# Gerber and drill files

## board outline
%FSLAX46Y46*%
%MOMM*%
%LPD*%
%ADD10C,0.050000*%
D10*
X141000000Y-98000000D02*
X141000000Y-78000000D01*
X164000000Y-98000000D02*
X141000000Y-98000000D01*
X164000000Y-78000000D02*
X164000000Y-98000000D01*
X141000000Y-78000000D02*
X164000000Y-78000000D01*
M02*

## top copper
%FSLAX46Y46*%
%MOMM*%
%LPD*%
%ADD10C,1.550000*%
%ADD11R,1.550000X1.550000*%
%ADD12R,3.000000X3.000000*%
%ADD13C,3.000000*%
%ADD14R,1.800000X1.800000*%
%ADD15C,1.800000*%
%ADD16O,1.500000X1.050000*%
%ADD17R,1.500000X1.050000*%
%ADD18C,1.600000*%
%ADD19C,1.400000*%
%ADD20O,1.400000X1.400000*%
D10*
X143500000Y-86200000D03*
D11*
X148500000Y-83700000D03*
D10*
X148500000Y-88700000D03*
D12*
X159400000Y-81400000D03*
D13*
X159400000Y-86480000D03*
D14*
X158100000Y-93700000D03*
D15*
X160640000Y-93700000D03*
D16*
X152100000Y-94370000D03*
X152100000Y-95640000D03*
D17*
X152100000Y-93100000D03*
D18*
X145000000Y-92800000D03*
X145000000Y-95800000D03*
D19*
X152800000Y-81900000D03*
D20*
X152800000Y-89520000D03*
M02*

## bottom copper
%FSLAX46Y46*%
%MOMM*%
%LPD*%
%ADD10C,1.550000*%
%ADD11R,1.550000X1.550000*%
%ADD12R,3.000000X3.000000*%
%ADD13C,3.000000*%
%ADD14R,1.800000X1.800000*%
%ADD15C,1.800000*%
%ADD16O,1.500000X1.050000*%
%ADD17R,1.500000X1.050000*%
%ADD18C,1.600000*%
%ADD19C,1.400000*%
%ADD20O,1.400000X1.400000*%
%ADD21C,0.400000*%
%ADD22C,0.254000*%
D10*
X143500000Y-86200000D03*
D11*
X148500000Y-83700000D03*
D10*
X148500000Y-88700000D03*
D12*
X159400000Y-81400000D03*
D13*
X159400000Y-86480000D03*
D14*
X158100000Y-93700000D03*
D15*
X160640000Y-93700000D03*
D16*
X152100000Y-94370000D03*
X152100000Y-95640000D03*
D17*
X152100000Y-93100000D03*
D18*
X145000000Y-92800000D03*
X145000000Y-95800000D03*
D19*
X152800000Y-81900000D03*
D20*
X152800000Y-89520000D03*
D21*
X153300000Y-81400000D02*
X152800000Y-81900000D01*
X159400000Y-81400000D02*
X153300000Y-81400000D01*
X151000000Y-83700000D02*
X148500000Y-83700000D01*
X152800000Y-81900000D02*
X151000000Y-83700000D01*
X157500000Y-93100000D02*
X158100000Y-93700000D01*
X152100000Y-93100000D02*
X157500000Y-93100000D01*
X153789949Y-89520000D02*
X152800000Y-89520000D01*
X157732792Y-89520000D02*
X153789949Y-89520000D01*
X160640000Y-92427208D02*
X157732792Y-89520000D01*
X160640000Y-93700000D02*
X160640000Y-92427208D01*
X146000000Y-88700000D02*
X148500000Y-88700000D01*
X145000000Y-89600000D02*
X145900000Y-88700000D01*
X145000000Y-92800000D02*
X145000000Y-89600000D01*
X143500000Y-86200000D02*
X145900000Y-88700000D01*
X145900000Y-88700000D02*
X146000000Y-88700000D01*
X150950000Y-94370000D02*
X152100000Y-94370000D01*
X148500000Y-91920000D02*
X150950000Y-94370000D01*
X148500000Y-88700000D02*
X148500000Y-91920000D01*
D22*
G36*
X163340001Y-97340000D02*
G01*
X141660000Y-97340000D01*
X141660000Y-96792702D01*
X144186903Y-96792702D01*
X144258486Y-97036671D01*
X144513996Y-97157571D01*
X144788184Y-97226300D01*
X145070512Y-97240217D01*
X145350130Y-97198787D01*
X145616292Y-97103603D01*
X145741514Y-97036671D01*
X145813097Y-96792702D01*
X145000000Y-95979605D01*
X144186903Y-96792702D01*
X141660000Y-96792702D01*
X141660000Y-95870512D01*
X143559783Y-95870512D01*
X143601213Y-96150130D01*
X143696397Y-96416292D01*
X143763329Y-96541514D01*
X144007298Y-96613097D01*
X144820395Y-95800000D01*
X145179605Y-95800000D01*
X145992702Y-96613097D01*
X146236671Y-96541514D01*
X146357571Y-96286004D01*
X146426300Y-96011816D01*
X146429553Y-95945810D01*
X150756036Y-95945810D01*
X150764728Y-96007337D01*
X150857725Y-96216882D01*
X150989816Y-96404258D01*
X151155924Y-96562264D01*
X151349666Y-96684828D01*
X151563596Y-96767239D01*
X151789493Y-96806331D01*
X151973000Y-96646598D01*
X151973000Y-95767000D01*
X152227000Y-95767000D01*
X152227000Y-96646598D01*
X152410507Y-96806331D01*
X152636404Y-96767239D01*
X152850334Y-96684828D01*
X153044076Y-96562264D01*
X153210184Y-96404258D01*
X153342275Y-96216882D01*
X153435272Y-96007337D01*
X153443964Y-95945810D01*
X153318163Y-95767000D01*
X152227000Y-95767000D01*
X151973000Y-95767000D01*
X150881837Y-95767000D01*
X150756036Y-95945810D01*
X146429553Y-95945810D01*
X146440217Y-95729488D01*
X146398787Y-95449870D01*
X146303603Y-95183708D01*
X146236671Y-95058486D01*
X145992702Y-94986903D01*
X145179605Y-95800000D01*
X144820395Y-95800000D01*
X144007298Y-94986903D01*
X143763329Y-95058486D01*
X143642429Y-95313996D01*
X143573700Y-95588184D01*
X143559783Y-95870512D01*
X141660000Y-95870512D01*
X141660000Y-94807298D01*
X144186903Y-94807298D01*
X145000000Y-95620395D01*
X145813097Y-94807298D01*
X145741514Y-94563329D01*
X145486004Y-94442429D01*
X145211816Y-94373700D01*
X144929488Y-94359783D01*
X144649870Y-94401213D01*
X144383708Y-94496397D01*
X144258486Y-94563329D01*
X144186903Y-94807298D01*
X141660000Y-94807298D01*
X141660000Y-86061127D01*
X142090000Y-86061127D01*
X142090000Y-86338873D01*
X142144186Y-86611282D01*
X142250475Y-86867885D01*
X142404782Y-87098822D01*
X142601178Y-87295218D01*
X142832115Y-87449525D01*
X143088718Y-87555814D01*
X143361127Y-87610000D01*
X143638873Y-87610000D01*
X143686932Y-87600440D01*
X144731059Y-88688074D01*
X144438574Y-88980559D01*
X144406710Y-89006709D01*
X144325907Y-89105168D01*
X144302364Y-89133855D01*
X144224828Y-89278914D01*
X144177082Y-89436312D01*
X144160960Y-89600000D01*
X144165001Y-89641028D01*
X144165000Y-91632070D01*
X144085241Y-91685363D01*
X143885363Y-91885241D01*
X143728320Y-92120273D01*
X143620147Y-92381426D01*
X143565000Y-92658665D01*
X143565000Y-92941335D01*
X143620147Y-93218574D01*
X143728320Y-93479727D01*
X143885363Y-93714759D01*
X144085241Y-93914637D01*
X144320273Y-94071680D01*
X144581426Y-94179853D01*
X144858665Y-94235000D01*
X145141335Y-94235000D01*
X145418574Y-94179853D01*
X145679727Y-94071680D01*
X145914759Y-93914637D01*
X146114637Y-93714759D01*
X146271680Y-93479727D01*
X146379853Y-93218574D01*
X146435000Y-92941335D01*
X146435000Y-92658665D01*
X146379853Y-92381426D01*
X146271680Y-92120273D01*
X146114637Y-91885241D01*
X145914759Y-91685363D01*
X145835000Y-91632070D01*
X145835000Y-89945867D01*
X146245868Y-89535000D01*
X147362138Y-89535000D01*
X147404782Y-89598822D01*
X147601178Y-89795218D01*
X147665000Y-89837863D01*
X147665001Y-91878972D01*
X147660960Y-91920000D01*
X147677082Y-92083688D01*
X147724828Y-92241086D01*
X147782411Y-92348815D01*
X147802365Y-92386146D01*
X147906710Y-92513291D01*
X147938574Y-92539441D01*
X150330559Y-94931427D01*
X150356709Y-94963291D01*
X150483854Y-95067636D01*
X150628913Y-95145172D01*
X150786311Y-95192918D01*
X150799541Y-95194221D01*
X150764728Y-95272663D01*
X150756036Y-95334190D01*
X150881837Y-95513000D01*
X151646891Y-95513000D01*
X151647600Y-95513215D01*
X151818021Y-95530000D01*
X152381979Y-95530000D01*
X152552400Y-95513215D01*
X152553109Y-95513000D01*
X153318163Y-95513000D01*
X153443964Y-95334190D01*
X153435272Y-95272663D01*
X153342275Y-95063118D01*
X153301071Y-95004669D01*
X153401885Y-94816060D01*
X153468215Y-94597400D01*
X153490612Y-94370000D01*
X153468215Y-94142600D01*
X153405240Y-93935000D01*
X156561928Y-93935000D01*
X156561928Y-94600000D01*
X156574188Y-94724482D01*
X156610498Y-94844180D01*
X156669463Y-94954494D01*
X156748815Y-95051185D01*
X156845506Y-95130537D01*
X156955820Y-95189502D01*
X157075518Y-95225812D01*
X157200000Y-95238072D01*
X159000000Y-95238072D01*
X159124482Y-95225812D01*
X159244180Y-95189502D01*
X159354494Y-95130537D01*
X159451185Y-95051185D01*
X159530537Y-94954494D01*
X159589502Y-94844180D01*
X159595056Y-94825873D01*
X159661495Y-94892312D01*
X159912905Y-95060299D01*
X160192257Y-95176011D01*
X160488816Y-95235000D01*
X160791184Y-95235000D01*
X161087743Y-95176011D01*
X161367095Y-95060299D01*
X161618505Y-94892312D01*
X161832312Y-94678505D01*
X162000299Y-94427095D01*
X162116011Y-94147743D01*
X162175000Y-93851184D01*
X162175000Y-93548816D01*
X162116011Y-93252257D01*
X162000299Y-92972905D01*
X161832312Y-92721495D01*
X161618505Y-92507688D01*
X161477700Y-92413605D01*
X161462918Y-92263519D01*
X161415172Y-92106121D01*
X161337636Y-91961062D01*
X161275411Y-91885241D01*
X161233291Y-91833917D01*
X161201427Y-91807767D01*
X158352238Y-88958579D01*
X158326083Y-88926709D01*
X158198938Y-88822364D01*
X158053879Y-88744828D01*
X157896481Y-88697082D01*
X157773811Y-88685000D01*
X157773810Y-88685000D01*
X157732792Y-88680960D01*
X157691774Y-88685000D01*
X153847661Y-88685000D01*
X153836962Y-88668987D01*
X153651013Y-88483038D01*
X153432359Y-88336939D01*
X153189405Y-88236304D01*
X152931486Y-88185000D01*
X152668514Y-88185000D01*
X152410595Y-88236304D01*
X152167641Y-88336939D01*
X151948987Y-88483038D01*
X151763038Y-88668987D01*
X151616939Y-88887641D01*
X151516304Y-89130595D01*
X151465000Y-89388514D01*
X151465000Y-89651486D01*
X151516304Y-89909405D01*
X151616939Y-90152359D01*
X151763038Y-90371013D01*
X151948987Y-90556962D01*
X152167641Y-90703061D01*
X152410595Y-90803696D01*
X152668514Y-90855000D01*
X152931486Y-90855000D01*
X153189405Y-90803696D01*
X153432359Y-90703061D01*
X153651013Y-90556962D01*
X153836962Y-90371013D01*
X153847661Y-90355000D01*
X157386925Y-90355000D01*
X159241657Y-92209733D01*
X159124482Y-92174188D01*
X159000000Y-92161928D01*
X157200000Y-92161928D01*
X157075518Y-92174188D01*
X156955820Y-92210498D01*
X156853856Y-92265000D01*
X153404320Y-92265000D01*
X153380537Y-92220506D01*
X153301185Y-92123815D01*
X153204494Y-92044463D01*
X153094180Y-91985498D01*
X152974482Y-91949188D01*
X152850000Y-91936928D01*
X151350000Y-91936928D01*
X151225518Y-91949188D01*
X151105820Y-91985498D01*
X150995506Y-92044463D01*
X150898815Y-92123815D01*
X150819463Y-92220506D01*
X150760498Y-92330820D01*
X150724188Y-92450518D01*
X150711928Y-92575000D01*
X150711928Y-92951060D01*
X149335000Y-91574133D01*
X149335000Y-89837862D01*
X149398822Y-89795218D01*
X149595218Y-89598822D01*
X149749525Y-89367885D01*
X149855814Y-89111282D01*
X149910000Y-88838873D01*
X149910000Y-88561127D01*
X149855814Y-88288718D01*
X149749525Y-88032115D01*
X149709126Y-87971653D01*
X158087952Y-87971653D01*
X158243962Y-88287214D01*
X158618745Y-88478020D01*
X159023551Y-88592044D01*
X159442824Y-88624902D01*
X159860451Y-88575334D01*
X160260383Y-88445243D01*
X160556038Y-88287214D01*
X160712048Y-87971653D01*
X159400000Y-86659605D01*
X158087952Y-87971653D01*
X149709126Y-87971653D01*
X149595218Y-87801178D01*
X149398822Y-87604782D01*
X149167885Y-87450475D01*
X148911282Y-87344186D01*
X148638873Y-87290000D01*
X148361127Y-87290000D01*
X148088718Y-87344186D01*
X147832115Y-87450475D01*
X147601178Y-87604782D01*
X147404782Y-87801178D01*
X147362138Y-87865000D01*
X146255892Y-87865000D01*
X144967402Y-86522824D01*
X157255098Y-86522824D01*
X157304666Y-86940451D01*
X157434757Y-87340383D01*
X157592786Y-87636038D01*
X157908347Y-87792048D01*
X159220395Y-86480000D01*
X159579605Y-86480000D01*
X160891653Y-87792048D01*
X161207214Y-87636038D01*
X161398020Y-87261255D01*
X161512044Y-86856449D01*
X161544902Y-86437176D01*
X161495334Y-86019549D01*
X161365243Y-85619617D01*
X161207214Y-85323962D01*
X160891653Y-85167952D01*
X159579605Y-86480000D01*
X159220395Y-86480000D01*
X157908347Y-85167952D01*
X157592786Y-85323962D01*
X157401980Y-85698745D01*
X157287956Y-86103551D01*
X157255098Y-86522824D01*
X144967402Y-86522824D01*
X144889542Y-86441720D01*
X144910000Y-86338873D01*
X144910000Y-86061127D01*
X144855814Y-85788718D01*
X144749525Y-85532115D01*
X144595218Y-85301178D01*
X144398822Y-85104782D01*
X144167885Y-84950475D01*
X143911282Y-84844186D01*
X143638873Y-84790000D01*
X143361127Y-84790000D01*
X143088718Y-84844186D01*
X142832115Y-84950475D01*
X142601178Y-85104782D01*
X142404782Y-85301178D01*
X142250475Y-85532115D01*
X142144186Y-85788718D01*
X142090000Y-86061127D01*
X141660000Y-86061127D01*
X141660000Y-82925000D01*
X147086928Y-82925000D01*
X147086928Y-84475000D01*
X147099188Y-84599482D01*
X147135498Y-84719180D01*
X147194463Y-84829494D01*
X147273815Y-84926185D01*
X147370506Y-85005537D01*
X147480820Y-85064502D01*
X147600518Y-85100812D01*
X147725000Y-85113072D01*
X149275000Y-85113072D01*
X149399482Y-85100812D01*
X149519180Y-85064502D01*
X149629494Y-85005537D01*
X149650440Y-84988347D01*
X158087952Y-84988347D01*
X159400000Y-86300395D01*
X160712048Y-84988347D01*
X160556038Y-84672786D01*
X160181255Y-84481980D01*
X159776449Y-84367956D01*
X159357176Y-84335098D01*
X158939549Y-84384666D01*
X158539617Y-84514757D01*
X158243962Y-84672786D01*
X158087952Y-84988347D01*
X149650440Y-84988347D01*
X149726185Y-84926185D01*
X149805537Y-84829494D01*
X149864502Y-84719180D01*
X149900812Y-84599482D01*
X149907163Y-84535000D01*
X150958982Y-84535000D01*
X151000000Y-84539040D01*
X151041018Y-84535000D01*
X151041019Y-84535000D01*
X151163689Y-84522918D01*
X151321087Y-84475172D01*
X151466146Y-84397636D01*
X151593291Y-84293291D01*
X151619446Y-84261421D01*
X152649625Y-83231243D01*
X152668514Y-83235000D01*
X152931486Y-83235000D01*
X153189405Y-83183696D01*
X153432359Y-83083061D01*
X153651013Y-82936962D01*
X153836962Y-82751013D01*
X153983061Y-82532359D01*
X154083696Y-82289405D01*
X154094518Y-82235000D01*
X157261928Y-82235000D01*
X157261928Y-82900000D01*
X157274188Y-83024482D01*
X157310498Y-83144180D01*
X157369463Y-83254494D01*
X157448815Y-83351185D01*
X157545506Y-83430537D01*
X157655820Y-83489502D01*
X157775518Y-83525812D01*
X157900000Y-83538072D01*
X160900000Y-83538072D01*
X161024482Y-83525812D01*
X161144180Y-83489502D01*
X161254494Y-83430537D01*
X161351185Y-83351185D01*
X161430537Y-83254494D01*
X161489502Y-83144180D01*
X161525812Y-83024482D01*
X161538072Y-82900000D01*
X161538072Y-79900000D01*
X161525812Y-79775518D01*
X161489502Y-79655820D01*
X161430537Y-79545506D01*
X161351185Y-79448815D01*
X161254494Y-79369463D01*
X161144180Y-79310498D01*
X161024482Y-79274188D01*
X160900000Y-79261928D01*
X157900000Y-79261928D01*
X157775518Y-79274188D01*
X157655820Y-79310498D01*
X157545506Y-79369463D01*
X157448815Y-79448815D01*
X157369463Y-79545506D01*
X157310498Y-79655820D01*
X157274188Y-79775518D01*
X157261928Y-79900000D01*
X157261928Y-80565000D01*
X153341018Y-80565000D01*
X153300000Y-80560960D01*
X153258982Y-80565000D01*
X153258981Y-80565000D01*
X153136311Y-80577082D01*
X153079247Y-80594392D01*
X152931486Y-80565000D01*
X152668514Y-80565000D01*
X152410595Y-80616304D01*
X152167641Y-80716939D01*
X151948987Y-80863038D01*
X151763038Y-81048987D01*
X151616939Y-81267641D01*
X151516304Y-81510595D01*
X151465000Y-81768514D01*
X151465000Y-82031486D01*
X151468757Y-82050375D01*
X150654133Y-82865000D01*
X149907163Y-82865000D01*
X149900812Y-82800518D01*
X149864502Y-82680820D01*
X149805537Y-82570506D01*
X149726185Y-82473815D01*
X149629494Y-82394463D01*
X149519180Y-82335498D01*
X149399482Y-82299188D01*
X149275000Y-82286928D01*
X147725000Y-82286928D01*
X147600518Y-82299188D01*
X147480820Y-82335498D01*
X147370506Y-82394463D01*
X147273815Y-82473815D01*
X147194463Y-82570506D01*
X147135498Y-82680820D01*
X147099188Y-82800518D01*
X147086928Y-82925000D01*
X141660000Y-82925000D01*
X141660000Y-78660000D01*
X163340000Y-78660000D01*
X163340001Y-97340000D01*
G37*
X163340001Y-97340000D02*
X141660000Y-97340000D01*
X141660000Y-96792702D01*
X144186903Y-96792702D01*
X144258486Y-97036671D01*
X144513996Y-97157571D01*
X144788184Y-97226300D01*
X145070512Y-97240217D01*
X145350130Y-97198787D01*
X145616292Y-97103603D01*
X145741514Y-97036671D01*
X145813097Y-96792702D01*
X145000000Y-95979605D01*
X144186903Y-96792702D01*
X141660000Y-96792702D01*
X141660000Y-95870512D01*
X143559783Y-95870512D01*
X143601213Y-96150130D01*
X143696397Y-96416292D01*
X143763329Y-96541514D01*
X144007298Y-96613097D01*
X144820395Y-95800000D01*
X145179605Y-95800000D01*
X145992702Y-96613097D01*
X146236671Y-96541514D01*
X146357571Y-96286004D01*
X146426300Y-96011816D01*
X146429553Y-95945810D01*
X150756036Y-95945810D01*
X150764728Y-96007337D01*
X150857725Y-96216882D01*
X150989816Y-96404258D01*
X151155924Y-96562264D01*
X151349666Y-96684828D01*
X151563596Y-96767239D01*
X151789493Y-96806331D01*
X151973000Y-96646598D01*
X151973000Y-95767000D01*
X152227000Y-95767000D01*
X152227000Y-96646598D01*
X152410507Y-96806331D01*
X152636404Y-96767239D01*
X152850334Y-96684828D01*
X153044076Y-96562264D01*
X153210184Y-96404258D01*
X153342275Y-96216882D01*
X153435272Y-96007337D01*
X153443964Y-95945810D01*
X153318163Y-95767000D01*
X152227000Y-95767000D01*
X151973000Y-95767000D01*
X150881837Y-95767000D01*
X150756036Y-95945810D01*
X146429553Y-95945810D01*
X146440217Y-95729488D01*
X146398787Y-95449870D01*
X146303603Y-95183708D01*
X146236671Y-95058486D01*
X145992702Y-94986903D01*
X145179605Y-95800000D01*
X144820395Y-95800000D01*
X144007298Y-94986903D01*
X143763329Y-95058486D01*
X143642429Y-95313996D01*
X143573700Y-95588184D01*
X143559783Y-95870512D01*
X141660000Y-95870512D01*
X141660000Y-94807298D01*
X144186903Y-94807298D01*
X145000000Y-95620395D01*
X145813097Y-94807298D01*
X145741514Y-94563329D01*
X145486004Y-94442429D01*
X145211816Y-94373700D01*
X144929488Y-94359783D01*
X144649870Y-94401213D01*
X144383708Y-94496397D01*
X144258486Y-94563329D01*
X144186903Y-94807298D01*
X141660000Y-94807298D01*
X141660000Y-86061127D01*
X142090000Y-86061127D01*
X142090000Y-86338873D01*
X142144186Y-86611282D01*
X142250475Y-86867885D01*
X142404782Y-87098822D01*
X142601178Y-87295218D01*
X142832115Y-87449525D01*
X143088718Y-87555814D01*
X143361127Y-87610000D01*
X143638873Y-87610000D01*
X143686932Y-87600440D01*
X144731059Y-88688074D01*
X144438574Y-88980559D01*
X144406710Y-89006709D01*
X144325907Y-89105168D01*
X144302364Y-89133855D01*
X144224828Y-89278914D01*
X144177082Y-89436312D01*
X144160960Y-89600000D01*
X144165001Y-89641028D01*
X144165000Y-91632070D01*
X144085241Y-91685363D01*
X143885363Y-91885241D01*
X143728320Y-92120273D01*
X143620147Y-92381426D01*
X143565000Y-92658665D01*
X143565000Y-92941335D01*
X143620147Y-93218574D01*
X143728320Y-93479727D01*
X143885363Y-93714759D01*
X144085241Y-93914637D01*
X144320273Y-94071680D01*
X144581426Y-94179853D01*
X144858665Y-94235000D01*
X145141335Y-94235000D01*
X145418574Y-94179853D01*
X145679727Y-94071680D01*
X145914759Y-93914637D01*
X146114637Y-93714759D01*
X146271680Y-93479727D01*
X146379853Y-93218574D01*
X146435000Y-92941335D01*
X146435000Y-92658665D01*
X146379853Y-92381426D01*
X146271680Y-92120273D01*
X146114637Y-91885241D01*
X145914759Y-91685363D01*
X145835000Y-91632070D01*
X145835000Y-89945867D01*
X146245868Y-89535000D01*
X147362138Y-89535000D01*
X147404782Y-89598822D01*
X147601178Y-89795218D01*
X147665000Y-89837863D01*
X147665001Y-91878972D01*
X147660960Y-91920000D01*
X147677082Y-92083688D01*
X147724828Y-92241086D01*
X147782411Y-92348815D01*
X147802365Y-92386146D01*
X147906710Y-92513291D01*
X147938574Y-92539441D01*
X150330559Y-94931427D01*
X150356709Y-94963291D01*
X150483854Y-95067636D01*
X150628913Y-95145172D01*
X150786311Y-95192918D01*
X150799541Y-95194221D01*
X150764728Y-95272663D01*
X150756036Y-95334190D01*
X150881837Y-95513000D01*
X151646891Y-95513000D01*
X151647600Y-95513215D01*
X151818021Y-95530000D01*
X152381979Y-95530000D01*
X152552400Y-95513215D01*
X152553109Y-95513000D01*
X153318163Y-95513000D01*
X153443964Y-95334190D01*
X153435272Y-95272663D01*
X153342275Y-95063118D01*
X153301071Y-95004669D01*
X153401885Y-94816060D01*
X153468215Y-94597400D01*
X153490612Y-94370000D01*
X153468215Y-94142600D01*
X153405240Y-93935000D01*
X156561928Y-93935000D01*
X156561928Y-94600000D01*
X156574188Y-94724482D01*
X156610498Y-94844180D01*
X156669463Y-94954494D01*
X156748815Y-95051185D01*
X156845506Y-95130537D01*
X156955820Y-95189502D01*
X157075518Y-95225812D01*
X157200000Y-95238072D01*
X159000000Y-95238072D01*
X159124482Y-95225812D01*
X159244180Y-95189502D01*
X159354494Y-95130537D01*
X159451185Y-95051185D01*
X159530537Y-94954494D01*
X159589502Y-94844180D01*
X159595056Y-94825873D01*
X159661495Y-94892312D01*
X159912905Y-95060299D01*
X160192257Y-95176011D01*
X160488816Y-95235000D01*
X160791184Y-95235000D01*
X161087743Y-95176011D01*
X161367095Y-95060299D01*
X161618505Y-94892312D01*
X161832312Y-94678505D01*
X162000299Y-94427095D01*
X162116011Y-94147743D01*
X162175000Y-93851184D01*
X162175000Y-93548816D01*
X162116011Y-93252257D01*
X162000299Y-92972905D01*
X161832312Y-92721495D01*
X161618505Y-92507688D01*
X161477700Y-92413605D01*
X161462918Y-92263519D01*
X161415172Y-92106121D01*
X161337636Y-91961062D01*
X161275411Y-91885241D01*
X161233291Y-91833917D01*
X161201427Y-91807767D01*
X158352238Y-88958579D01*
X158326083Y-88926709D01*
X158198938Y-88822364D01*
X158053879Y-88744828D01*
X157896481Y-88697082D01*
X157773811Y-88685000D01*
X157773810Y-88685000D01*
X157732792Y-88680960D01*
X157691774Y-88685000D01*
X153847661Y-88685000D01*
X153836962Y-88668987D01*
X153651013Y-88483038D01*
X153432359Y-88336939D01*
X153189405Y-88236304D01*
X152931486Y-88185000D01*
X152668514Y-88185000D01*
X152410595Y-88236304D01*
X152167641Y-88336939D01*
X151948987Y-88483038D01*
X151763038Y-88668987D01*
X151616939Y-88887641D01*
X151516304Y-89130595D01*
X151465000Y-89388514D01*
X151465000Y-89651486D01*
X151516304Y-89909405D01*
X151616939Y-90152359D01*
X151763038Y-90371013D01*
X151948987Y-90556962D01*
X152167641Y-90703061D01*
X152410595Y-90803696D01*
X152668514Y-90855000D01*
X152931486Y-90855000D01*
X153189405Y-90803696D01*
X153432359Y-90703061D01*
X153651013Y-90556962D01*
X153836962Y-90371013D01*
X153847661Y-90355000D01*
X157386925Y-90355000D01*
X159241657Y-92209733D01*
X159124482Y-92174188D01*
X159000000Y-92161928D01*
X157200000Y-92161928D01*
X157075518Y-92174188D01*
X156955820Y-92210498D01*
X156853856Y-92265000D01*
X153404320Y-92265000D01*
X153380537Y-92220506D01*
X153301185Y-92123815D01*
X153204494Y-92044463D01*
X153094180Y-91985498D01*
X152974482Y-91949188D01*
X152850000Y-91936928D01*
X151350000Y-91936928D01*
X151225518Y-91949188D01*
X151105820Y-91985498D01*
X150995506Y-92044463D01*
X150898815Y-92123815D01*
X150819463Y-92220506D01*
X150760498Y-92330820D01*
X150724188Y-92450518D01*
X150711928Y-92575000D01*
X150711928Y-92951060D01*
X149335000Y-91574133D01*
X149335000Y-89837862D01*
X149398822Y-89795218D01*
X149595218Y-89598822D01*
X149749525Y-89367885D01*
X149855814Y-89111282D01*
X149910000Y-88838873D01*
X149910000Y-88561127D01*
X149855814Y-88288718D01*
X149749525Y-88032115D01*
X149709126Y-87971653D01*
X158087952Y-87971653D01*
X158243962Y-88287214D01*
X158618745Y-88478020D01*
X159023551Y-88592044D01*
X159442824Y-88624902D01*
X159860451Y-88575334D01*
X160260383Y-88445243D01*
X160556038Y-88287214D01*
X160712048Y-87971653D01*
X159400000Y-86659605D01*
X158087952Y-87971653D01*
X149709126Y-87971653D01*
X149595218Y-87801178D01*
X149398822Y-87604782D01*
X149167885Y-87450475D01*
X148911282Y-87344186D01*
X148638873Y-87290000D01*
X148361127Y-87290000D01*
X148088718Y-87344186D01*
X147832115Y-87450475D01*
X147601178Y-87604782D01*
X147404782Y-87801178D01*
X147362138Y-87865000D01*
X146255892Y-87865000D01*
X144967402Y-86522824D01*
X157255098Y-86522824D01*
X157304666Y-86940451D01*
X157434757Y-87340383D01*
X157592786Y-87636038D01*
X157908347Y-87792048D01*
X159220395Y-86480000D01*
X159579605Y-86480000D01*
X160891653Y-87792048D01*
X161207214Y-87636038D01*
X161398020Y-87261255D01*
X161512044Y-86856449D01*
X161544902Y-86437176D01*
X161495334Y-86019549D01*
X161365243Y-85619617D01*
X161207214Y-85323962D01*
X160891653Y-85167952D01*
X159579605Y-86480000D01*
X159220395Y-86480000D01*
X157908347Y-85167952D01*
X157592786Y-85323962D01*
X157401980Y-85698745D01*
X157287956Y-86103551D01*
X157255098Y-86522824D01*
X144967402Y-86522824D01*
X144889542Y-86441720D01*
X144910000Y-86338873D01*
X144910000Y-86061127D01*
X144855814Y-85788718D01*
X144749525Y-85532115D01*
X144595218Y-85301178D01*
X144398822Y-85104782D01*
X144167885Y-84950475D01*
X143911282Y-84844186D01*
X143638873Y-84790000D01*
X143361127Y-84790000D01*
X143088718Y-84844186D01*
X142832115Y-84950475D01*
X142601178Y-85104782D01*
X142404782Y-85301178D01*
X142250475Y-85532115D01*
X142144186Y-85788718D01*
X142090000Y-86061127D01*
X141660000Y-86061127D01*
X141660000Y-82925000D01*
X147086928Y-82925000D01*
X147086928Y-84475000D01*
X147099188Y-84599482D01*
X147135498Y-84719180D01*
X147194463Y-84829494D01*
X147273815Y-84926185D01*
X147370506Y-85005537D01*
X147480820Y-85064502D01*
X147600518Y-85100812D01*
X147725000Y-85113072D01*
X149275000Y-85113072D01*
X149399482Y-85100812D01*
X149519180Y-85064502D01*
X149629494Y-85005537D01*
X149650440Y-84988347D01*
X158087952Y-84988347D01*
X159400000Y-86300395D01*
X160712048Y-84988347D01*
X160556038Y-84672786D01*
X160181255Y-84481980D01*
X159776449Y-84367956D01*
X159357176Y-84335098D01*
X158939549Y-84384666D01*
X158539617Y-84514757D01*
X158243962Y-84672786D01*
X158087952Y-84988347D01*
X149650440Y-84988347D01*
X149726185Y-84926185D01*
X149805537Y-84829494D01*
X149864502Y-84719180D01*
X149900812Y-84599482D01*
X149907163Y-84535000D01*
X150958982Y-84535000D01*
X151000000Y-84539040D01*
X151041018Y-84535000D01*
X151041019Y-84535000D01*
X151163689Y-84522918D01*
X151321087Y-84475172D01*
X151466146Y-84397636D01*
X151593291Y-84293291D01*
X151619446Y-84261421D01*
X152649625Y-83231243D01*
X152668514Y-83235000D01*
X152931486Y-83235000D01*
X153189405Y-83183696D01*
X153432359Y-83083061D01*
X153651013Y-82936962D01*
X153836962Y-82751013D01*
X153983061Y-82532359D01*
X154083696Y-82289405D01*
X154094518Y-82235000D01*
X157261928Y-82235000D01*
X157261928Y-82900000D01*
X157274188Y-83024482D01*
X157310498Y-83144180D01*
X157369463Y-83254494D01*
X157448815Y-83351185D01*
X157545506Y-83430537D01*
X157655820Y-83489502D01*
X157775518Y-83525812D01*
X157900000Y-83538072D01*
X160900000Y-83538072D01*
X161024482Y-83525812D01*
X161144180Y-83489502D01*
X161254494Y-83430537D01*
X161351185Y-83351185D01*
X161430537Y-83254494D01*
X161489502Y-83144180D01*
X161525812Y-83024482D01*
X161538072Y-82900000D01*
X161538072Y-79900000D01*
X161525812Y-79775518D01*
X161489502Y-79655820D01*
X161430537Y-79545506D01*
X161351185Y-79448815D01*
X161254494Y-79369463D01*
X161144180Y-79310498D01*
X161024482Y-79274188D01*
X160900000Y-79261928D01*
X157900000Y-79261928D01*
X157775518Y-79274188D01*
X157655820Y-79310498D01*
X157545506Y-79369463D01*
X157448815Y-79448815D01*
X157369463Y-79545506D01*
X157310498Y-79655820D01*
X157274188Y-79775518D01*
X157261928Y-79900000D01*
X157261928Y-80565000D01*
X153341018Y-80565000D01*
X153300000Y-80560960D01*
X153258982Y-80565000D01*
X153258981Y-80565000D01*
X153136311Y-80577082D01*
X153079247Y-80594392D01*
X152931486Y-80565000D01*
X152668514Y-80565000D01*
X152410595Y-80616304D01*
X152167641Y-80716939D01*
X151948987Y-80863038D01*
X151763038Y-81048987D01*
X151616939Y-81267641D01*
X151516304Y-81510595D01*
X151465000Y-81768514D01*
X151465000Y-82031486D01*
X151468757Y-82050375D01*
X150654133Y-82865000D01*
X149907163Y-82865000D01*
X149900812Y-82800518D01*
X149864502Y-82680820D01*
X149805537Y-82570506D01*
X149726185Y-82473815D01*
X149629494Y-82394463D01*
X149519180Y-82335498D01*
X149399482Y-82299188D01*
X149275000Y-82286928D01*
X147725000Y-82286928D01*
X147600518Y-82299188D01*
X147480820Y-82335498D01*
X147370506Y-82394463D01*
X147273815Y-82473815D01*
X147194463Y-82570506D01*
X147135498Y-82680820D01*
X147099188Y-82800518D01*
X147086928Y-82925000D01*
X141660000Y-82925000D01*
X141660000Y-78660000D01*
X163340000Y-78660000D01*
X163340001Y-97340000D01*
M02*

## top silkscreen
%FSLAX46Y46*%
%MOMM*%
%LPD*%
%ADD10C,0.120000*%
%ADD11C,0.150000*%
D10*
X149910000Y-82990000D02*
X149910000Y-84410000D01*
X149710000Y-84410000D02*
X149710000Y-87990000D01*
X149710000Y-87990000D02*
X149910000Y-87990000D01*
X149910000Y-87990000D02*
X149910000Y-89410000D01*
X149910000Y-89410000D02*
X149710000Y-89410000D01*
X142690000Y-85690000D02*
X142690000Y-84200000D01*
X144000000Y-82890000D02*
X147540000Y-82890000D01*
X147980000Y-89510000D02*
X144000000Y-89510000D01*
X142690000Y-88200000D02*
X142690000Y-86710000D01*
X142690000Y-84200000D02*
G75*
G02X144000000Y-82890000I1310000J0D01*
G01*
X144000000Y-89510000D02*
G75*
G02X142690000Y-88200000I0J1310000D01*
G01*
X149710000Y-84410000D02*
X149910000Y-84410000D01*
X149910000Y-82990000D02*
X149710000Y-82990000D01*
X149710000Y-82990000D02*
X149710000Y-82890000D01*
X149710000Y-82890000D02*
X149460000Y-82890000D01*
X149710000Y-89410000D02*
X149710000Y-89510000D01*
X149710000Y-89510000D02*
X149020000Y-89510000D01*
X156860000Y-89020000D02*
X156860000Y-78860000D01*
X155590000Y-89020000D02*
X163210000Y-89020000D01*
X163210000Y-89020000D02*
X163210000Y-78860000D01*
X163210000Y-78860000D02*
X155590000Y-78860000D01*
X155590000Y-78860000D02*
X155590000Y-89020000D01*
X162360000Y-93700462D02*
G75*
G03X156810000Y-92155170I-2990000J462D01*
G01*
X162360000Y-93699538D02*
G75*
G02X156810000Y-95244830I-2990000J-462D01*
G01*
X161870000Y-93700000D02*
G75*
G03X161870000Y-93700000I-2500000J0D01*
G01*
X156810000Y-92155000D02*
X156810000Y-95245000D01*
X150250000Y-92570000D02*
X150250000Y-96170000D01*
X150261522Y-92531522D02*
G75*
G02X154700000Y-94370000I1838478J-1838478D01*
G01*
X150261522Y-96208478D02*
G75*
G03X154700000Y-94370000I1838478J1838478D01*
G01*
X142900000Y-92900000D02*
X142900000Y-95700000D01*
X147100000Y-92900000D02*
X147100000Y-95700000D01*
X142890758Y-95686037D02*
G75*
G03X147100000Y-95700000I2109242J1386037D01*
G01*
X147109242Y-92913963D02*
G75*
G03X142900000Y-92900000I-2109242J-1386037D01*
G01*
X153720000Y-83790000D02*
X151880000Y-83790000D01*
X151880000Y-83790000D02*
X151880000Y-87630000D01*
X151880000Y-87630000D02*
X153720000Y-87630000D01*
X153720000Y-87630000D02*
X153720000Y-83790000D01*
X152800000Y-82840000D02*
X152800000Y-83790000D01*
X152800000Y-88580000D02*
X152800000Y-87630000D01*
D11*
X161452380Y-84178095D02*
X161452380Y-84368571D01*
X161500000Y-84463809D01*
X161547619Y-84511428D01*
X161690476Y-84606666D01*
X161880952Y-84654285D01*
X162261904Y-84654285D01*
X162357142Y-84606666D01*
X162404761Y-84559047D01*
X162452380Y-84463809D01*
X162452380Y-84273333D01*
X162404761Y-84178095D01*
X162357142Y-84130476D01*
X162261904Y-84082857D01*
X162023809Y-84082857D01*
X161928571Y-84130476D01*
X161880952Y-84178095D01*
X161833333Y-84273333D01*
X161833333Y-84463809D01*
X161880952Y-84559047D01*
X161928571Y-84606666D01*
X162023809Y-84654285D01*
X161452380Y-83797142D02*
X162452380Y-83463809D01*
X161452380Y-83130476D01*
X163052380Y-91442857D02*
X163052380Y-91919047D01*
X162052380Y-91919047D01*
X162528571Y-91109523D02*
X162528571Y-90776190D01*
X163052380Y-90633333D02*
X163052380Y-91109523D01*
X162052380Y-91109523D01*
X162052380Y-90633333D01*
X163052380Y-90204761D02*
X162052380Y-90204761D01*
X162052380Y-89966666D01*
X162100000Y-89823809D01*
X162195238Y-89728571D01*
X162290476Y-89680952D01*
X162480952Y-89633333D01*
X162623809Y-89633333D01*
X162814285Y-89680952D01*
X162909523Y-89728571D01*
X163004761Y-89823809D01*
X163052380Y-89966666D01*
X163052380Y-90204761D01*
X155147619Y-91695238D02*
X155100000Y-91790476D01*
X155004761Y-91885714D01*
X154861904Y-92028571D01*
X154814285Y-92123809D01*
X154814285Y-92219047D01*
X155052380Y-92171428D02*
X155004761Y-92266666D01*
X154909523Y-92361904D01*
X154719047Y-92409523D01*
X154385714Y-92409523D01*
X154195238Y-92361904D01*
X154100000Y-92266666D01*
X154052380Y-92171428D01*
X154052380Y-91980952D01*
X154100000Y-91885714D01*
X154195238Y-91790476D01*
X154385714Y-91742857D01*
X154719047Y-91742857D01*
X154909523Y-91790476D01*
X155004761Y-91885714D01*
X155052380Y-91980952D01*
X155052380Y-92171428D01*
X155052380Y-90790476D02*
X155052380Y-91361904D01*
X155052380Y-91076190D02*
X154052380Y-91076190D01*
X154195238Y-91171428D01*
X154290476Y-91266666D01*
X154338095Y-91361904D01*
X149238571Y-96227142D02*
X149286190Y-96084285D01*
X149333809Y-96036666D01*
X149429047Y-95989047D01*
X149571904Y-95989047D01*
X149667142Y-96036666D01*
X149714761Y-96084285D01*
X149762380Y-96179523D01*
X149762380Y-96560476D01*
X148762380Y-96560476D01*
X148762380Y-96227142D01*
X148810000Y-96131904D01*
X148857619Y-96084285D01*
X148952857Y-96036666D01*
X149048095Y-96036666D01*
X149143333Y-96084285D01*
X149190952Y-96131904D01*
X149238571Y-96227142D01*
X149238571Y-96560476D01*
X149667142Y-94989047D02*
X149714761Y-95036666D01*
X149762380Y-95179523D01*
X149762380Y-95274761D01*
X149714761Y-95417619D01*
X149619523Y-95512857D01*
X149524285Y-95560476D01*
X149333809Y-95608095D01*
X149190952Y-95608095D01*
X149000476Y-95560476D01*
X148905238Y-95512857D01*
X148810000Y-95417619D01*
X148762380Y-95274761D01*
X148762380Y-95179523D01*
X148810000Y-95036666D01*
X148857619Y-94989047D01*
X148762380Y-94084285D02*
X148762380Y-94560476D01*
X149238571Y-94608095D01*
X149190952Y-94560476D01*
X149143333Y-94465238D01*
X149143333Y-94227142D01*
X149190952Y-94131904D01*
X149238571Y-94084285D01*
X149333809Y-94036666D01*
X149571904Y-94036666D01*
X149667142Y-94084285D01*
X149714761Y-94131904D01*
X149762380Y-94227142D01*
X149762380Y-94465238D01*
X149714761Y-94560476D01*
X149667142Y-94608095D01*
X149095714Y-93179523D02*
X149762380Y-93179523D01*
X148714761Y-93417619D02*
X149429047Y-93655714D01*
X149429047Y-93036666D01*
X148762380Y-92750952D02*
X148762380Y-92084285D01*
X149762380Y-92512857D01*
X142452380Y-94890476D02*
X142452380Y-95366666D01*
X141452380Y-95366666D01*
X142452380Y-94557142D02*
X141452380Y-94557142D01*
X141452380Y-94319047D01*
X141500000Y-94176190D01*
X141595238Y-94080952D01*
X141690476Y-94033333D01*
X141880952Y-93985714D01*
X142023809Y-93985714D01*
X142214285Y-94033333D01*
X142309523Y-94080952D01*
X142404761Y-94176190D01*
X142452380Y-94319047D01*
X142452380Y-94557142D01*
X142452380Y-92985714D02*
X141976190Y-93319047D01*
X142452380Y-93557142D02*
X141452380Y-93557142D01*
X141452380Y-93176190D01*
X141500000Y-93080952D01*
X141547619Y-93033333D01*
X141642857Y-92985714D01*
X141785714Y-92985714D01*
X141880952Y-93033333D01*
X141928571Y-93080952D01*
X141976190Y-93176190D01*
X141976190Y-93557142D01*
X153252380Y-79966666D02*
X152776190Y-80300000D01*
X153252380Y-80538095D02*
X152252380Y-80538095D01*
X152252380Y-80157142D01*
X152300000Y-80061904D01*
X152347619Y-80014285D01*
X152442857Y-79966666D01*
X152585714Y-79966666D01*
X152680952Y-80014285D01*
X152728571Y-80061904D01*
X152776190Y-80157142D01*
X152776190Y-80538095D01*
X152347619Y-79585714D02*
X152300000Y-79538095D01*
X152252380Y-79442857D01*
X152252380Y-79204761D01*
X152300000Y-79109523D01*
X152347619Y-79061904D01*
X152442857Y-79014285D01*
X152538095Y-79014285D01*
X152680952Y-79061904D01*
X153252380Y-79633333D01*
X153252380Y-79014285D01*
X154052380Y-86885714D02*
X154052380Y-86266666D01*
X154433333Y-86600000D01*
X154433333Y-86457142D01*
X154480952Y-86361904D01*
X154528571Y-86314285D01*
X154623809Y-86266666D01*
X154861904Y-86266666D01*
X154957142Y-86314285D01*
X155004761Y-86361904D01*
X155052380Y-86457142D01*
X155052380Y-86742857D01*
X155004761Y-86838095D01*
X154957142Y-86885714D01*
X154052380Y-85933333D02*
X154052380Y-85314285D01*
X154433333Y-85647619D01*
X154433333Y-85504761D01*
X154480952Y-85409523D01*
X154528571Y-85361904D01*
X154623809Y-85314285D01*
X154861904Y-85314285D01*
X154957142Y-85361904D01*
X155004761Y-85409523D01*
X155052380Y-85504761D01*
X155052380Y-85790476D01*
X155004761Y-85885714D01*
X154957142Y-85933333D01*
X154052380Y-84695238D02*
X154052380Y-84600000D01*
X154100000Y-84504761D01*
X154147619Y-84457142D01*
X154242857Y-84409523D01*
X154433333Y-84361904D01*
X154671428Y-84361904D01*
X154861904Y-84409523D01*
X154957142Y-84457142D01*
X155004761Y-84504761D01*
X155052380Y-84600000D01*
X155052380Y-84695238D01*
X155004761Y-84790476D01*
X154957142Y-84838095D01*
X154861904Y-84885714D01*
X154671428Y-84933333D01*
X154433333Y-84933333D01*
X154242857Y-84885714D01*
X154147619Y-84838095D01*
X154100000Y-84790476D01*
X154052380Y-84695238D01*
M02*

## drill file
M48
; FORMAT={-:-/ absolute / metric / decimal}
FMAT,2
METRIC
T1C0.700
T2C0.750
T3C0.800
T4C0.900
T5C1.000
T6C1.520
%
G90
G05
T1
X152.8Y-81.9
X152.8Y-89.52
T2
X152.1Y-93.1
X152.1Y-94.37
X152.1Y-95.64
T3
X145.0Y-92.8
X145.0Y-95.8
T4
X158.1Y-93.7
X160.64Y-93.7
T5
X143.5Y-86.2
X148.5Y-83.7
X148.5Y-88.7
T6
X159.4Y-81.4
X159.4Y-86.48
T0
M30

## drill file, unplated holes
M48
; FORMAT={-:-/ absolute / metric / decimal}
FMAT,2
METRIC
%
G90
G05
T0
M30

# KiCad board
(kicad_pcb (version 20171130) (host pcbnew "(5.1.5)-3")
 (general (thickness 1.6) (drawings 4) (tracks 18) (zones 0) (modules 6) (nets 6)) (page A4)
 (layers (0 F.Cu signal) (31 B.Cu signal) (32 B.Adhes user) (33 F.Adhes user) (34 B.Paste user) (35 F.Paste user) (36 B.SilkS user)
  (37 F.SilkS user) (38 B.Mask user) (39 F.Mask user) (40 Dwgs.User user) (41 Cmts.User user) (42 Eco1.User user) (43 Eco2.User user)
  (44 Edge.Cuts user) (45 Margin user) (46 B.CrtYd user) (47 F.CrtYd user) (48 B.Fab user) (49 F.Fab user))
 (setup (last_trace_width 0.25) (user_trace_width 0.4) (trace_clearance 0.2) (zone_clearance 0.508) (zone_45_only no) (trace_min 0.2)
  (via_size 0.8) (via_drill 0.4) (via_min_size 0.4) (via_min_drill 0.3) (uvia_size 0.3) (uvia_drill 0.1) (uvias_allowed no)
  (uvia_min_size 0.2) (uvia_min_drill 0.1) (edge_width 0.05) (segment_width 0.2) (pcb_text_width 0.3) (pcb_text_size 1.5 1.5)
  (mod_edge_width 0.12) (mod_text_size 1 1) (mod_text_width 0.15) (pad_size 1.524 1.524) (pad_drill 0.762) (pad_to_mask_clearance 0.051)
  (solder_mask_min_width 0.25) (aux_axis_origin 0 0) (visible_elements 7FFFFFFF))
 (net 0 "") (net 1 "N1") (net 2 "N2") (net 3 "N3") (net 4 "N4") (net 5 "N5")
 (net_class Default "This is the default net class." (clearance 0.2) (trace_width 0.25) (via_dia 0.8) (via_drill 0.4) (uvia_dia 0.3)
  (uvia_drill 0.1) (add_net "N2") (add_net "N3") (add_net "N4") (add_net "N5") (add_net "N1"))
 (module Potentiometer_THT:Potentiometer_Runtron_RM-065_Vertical (layer F.Cu) (at 148.5 83.7 270)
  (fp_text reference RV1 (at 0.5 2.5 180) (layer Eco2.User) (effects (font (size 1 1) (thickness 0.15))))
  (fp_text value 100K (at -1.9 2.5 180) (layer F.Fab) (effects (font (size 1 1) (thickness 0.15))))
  (fp_line (start -0.71 -1.41) (end 0.71 -1.41) (layer F.SilkS) (width 0.12))
  (fp_line (start 0.71 -1.21) (end 4.29 -1.21) (layer F.SilkS) (width 0.12))
  (fp_line (start 4.29 -1.21) (end 4.29 -1.41) (layer F.SilkS) (width 0.12))
  (fp_line (start 4.29 -1.41) (end 5.71 -1.41) (layer F.SilkS) (width 0.12))
  (fp_line (start 5.71 -1.41) (end 5.71 -1.21) (layer F.SilkS) (width 0.12))
  (fp_line (start 1.99 5.81) (end 0.5 5.81) (layer F.SilkS) (width 0.12))
  (fp_line (start -0.81 4.5) (end -0.81 0.96) (layer F.SilkS) (width 0.12))
  (fp_line (start 5.81 0.52) (end 5.81 4.5) (layer F.SilkS) (width 0.12))
  (fp_line (start 4.5 5.81) (end 3.01 5.81) (layer F.SilkS) (width 0.12))
  (fp_arc (start 0.5 4.5) (end -0.81 4.5) (angle -90) (layer F.SilkS) (width 0.12))
  (fp_arc (start 4.5 4.5) (end 4.5 5.81) (angle -90) (layer F.SilkS) (width 0.12))
  (fp_line (start 0.71 -1.21) (end 0.71 -1.41) (layer F.SilkS) (width 0.12))
  (fp_line (start -0.71 -1.41) (end -0.71 -1.21) (layer F.SilkS) (width 0.12))
  (fp_line (start -0.71 -1.21) (end -0.81 -1.21) (layer F.SilkS) (width 0.12))
  (fp_line (start -0.81 -1.21) (end -0.81 -0.96) (layer F.SilkS) (width 0.12))
  (fp_line (start 5.71 -1.21) (end 5.81 -1.21) (layer F.SilkS) (width 0.12))
  (fp_line (start 5.81 -1.21) (end 5.81 -0.52) (layer F.SilkS) (width 0.12))
  (pad 2 thru_hole circle (at 2.5 5 270) (size 1.55 1.55) (drill 1) (layers *.Cu *.Mask) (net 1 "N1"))
  (pad 1 thru_hole rect (at 0 0 270) (size 1.55 1.55) (drill 1) (layers *.Cu *.Mask) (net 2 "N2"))
  (pad 3 thru_hole circle (at 5 0 270) (size 1.55 1.55) (drill 1) (layers *.Cu *.Mask) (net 1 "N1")))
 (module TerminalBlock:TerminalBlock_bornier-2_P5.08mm (layer F.Cu) (at 159.4 81.4 270)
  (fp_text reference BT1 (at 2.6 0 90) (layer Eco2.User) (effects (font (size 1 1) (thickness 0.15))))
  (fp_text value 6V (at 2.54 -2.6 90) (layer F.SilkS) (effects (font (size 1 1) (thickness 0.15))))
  (fp_line (start 7.62 2.54) (end -2.54 2.54) (layer F.SilkS) (width 0.12))
  (fp_line (start 7.62 3.81) (end 7.62 -3.81) (layer F.SilkS) (width 0.12))
  (fp_line (start 7.62 -3.81) (end -2.54 -3.81) (layer F.SilkS) (width 0.12))
  (fp_line (start -2.54 -3.81) (end -2.54 3.81) (layer F.SilkS) (width 0.12))
  (fp_line (start -2.54 3.81) (end 7.62 3.81) (layer F.SilkS) (width 0.12))
  (pad 1 thru_hole rect (at 0 0 270) (size 3 3) (drill 1.52) (layers *.Cu *.Mask) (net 2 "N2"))
  (pad 2 thru_hole circle (at 5.08 0 270) (size 3 3) (drill 1.52) (layers *.Cu *.Mask) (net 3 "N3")))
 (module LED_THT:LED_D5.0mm (layer F.Cu) (at 158.1 93.7)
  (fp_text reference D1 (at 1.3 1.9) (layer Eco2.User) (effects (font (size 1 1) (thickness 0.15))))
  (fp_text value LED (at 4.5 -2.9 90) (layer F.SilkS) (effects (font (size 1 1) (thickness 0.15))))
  (fp_arc (start 1.27 0) (end -1.29 -1.54483) (angle 148.9) (layer F.SilkS) (width 0.12))
  (fp_arc (start 1.27 0) (end -1.29 1.54483) (angle -148.9) (layer F.SilkS) (width 0.12))
  (fp_circle (center 1.27 0) (end 3.77 0) (layer F.SilkS) (width 0.12))
  (fp_line (start -1.29 -1.545) (end -1.29 1.545) (layer F.SilkS) (width 0.12))
  (pad 1 thru_hole rect (at 0 0) (size 1.8 1.8) (drill 0.9) (layers *.Cu *.Mask) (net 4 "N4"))
  (pad 2 thru_hole circle (at 2.54 0) (size 1.8 1.8) (drill 0.9) (layers *.Cu *.Mask) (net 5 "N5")))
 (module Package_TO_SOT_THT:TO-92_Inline (layer F.Cu) (at 152.1 93.1 270)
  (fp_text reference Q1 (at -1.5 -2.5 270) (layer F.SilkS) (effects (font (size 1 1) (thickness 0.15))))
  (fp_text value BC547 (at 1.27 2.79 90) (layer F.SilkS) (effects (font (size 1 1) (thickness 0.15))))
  (fp_line (start -0.53 1.85) (end 3.07 1.85) (layer F.SilkS) (width 0.12))
  (fp_arc (start 1.27 0) (end 1.27 -2.6) (angle -135) (layer F.SilkS) (width 0.12))
  (fp_arc (start 1.27 0) (end 1.27 -2.6) (angle 135) (layer F.SilkS) (width 0.12))
  (pad 2 thru_hole oval (at 1.27 0 270) (size 1.05 1.5) (drill 0.75) (layers *.Cu *.Mask) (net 1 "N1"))
  (pad 3 thru_hole oval (at 2.54 0 270) (size 1.05 1.5) (drill 0.75) (layers *.Cu *.Mask) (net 3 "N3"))
  (pad 1 thru_hole rect (at 0 0 270) (size 1.05 1.5) (drill 0.75) (layers *.Cu *.Mask) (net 4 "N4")))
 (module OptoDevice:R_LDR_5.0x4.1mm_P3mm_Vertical (layer F.Cu) (at 145 92.8 270)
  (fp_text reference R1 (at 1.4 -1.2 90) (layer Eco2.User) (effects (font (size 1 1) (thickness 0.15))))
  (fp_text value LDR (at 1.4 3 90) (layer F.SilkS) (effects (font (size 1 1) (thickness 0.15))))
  (fp_line (start 0.1 2.1) (end 2.9 2.1) (layer F.SilkS) (width 0.12))
  (fp_line (start 0.1 -2.1) (end 2.9 -2.1) (layer F.SilkS) (width 0.12))
  (fp_arc (start 1.5 0) (end 2.9 -2.1) (angle 113) (layer F.SilkS) (width 0.12))
  (fp_arc (start 1.5 0) (end 0.1 2.1) (angle 113) (layer F.SilkS) (width 0.12))
  (pad 1 thru_hole circle (at 0 0 270) (size 1.6 1.6) (drill 0.8) (layers *.Cu *.Mask) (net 1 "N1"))
  (pad 2 thru_hole circle (at 3 0 270) (size 1.6 1.6) (drill 0.8) (layers *.Cu *.Mask) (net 3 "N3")))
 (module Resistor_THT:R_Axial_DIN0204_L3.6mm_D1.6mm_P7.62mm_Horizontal (layer F.Cu) (at 152.8 81.9 270)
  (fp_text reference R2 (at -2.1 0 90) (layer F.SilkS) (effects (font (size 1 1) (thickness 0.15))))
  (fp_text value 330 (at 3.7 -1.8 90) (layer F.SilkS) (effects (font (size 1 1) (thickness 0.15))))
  (fp_line (start 1.89 -0.92) (end 1.89 0.92) (layer F.SilkS) (width 0.12))
  (fp_line (start 1.89 0.92) (end 5.73 0.92) (layer F.SilkS) (width 0.12))
  (fp_line (start 5.73 0.92) (end 5.73 -0.92) (layer F.SilkS) (width 0.12))
  (fp_line (start 5.73 -0.92) (end 1.89 -0.92) (layer F.SilkS) (width 0.12))
  (fp_line (start 0.94 0) (end 1.89 0) (layer F.SilkS) (width 0.12))
  (fp_line (start 6.68 0) (end 5.73 0) (layer F.SilkS) (width 0.12))
  (pad 1 thru_hole circle (at 0 0 270) (size 1.4 1.4) (drill 0.7) (layers *.Cu *.Mask) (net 2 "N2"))
  (pad 2 thru_hole oval (at 7.62 0 270) (size 1.4 1.4) (drill 0.7) (layers *.Cu *.Mask) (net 5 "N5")))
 (gr_line (start 141 98) (end 141 78) (layer Edge.Cuts) (width 0.05))
 (gr_line (start 164 98) (end 141 98) (layer Edge.Cuts) (width 0.05))
 (gr_line (start 164 78) (end 164 98) (layer Edge.Cuts) (width 0.05))
 (gr_line (start 141 78) (end 164 78) (layer Edge.Cuts) (width 0.05))
 (segment (start 153.3 81.4) (end 152.8 81.9) (width 0.4) (layer B.Cu) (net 2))
 (segment (start 159.4 81.4) (end 153.3 81.4) (width 0.4) (layer B.Cu) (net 2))
 (segment (start 151 83.7) (end 148.5 83.7) (width 0.4) (layer B.Cu) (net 2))
 (segment (start 152.8 81.9) (end 151 83.7) (width 0.4) (layer B.Cu) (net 2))
 (segment (start 157.5 93.1) (end 158.1 93.7) (width 0.4) (layer B.Cu) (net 4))
 (segment (start 152.1 93.1) (end 157.5 93.1) (width 0.4) (layer B.Cu) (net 4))
 (segment (start 153.789949 89.52) (end 152.8 89.52) (width 0.4) (layer B.Cu) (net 5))
 (segment (start 157.732792 89.52) (end 153.789949 89.52) (width 0.4) (layer B.Cu) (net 5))
 (segment (start 160.64 92.427208) (end 157.732792 89.52) (width 0.4) (layer B.Cu) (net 5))
 (segment (start 160.64 93.7) (end 160.64 92.427208) (width 0.4) (layer B.Cu) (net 5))
 (segment (start 146 88.7) (end 148.5 88.7) (width 0.4) (layer B.Cu) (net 1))
 (segment (start 145 89.6) (end 145.9 88.7) (width 0.4) (layer B.Cu) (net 1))
 (segment (start 145 92.8) (end 145 89.6) (width 0.4) (layer B.Cu) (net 1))
 (segment (start 143.5 86.2) (end 145.9 88.7) (width 0.4) (layer B.Cu) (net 1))
 (segment (start 145.9 88.7) (end 146 88.7) (width 0.4) (layer B.Cu) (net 1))
 (segment (start 150.95 94.37) (end 152.1 94.37) (width 0.4) (layer B.Cu) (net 1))
 (segment (start 148.5 91.92) (end 150.95 94.37) (width 0.4) (layer B.Cu) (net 1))
 (segment (start 148.5 88.7) (end 148.5 91.92) (width 0.4) (layer B.Cu) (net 1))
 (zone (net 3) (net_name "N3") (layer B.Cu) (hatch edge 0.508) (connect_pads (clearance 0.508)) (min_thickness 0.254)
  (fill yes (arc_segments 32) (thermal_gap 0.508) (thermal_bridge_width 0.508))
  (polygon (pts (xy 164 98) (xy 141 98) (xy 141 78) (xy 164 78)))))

